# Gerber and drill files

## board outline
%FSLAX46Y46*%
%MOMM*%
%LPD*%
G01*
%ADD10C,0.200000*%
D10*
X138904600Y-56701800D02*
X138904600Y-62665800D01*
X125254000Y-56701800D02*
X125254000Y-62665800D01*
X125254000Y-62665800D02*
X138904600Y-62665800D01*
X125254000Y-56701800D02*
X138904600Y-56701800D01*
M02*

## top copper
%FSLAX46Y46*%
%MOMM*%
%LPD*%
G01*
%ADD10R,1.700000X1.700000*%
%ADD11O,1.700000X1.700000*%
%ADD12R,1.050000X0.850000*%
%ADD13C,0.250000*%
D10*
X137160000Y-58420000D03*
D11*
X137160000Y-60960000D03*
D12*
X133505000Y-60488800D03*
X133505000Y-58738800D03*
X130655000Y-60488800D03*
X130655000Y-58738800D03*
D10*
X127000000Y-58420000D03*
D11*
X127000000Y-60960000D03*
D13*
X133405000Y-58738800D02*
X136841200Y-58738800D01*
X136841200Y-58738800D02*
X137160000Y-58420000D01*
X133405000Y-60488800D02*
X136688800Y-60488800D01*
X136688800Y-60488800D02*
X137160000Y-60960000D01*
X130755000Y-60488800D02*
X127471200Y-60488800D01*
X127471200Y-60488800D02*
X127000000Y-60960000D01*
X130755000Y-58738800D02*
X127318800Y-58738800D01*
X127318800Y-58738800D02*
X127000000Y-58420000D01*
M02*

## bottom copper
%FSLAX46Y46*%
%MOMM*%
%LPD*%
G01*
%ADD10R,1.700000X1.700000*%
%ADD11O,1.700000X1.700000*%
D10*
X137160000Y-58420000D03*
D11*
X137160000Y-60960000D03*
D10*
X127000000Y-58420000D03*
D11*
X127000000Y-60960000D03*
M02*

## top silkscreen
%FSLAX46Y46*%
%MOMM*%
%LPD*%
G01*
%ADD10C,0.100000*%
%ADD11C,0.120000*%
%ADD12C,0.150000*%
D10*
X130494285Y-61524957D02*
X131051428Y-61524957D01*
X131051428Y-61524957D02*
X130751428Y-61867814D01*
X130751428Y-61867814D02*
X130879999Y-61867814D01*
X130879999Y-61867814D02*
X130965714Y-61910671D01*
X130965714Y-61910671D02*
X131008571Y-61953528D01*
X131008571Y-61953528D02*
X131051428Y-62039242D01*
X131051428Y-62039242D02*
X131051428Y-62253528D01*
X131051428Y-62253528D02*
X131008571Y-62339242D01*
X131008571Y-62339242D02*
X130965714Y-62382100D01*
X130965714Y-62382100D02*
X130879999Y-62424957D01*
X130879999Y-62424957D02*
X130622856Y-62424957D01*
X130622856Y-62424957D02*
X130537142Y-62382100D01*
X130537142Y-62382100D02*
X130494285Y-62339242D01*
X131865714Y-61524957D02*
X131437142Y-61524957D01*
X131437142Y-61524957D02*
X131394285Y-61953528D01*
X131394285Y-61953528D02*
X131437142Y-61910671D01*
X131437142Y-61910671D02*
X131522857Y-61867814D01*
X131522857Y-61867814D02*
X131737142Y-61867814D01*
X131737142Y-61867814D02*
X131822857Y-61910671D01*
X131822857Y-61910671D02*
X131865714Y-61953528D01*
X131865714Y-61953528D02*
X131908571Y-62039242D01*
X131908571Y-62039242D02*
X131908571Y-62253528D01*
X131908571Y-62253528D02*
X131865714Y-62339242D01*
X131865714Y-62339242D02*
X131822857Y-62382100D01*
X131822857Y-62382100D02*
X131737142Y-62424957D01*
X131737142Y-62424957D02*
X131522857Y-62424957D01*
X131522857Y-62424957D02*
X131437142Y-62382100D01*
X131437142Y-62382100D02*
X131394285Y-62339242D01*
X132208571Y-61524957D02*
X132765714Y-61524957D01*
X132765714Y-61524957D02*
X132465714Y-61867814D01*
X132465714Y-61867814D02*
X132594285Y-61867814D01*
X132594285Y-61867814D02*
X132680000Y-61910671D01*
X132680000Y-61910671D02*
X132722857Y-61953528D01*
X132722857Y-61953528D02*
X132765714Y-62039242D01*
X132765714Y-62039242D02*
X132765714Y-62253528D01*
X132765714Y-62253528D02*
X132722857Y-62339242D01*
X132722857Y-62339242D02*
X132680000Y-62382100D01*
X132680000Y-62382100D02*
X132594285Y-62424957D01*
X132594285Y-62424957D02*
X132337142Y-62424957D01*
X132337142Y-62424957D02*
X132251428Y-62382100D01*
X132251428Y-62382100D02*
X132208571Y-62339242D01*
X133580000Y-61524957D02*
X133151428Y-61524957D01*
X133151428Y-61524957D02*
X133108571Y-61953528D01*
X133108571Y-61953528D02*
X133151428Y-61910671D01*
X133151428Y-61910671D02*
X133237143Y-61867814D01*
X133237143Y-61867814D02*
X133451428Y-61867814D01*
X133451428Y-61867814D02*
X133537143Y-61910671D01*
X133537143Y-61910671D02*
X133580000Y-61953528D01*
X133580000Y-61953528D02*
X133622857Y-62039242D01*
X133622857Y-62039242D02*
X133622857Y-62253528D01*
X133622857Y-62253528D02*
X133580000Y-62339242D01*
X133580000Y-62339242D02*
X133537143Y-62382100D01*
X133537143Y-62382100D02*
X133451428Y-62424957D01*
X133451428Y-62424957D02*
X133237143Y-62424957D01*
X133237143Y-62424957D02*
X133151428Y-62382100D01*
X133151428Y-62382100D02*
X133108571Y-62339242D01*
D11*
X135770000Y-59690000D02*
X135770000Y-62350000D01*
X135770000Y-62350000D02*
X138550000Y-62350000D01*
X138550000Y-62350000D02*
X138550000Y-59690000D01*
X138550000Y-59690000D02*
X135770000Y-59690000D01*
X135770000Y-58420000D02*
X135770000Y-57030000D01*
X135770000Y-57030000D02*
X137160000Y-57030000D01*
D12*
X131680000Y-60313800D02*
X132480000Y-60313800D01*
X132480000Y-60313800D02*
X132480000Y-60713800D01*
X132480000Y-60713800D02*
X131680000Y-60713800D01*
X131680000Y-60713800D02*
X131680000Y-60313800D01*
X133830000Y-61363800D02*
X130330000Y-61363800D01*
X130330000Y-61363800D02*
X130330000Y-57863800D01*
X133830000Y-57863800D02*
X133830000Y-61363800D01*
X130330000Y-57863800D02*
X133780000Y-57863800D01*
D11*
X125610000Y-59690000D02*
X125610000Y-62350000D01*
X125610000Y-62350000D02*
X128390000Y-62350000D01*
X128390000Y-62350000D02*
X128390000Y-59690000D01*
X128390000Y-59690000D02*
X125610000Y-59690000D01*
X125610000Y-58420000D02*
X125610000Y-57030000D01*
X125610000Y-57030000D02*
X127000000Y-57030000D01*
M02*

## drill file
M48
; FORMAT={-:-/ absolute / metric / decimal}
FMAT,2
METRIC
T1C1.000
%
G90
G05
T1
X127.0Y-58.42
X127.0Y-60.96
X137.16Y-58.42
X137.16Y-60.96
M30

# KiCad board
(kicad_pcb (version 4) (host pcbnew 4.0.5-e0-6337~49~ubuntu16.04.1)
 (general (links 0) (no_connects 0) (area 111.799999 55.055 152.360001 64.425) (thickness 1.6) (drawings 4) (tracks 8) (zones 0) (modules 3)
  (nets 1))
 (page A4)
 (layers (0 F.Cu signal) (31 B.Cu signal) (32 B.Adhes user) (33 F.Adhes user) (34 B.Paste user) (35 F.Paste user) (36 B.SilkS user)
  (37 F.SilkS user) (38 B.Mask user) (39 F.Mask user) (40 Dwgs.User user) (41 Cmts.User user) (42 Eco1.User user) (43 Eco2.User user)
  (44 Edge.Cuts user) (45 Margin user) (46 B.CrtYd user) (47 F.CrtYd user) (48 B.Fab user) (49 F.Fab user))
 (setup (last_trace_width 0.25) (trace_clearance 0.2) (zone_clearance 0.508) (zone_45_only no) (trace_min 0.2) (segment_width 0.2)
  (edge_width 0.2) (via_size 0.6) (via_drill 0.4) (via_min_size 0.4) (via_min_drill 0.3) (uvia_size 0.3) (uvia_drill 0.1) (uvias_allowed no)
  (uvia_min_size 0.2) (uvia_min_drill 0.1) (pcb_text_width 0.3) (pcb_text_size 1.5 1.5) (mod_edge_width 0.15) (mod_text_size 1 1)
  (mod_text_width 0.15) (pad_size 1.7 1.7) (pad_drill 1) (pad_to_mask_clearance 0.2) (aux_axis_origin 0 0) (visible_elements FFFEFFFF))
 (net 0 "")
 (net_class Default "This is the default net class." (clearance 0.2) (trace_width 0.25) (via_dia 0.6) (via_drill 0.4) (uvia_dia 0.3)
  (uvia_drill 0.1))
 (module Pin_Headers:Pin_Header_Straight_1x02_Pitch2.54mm (layer F.Cu) (at 137.16 58.42)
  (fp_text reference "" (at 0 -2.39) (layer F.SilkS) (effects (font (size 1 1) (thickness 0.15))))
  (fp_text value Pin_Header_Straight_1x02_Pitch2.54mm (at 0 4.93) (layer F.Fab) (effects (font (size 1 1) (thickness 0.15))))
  (fp_line (start -1.39 1.27) (end -1.39 3.93) (layer F.SilkS) (width 0.12))
  (fp_line (start -1.39 3.93) (end 1.39 3.93) (layer F.SilkS) (width 0.12))
  (fp_line (start 1.39 3.93) (end 1.39 1.27) (layer F.SilkS) (width 0.12))
  (fp_line (start 1.39 1.27) (end -1.39 1.27) (layer F.SilkS) (width 0.12))
  (fp_line (start -1.39 0) (end -1.39 -1.39) (layer F.SilkS) (width 0.12))
  (fp_line (start -1.39 -1.39) (end 0 -1.39) (layer F.SilkS) (width 0.12))
  (pad 1 thru_hole rect (at 0 0) (size 1.7 1.7) (drill 1) (layers *.Cu *.Mask))
  (pad 2 thru_hole oval (at 0 2.54) (size 1.7 1.7) (drill 1) (layers *.Cu *.Mask)))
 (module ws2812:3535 (layer F.Cu) (at 132.08 59.6138)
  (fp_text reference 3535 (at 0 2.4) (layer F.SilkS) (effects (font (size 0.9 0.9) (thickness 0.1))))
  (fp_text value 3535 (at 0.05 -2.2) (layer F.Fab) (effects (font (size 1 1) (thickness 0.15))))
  (fp_line (start -0.4 0.7) (end 0.4 0.7) (layer F.SilkS) (width 0.15))
  (fp_line (start 0.4 0.7) (end 0.4 1.1) (layer F.SilkS) (width 0.15))
  (fp_line (start 0.4 1.1) (end -0.4 1.1) (layer F.SilkS) (width 0.15))
  (fp_line (start -0.4 1.1) (end -0.4 0.7) (layer F.SilkS) (width 0.15))
  (fp_line (start 1.75 1.75) (end -1.75 1.75) (layer F.SilkS) (width 0.15))
  (fp_line (start -1.75 1.75) (end -1.75 -1.75) (layer F.SilkS) (width 0.15))
  (fp_line (start 1.75 -1.75) (end 1.75 1.75) (layer F.SilkS) (width 0.15))
  (fp_line (start -1.75 -1.75) (end 1.7 -1.75) (layer F.SilkS) (width 0.15))
  (pad IN smd rect (at 1.325 0.875) (size 1.05 0.85) (drill (offset 0.1 0)) (layers F.Cu F.Paste F.Mask))
  (pad VDD smd rect (at 1.325 -0.875) (size 1.05 0.85) (drill (offset 0.1 0)) (layers F.Cu F.Paste F.Mask))
  (pad GND smd rect (at -1.325 0.875) (size 1.05 0.85) (drill (offset -0.1 0)) (layers F.Cu F.Paste F.Mask))
  (pad OUT smd rect (at -1.325 -0.875) (size 1.05 0.85) (drill (offset -0.1 0)) (layers F.Cu F.Paste F.Mask)))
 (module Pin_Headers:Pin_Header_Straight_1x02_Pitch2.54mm (layer F.Cu) (at 127 58.42)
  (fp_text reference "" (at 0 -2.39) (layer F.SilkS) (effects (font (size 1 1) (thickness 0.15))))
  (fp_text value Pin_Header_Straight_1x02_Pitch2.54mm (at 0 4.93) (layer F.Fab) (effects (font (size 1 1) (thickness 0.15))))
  (fp_line (start -1.39 1.27) (end -1.39 3.93) (layer F.SilkS) (width 0.12))
  (fp_line (start -1.39 3.93) (end 1.39 3.93) (layer F.SilkS) (width 0.12))
  (fp_line (start 1.39 3.93) (end 1.39 1.27) (layer F.SilkS) (width 0.12))
  (fp_line (start 1.39 1.27) (end -1.39 1.27) (layer F.SilkS) (width 0.12))
  (fp_line (start -1.39 0) (end -1.39 -1.39) (layer F.SilkS) (width 0.12))
  (fp_line (start -1.39 -1.39) (end 0 -1.39) (layer F.SilkS) (width 0.12))
  (pad 1 thru_hole rect (at 0 0) (size 1.7 1.7) (drill 1) (layers *.Cu *.Mask))
  (pad 2 thru_hole oval (at 0 2.54) (size 1.7 1.7) (drill 1) (layers *.Cu *.Mask)))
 (gr_line (start 138.9046 56.7018) (end 138.9046 62.6658) (angle 90) (layer Edge.Cuts) (width 0.2))
 (gr_line (start 125.254 56.7018) (end 125.254 62.6658) (angle 90) (layer Edge.Cuts) (width 0.2))
 (gr_line (start 125.254 62.6658) (end 138.9046 62.6658) (angle 90) (layer Edge.Cuts) (width 0.2))
 (gr_line (start 125.254 56.7018) (end 138.9046 56.7018) (angle 90) (layer Edge.Cuts) (width 0.2))
 (segment (start 133.405 58.7388) (end 136.8412 58.7388) (width 0.25) (layer F.Cu) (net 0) (status C00000))
 (segment (start 136.8412 58.7388) (end 137.16 58.42) (width 0.25) (layer F.Cu) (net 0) (status C00000))
 (segment (start 133.405 60.4888) (end 136.6888 60.4888) (width 0.25) (layer F.Cu) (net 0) (status C00000))
 (segment (start 136.6888 60.4888) (end 137.16 60.96) (width 0.25) (layer F.Cu) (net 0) (status C00000))
 (segment (start 130.755 60.4888) (end 127.4712 60.4888) (width 0.25) (layer F.Cu) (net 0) (status C00000))
 (segment (start 127.4712 60.4888) (end 127 60.96) (width 0.25) (layer F.Cu) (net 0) (status C00000))
 (segment (start 130.755 58.7388) (end 127.3188 58.7388) (width 0.25) (layer F.Cu) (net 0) (status C00000))
 (segment (start 127.3188 58.7388) (end 127 58.42) (width 0.25) (layer F.Cu) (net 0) (status C00000)))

